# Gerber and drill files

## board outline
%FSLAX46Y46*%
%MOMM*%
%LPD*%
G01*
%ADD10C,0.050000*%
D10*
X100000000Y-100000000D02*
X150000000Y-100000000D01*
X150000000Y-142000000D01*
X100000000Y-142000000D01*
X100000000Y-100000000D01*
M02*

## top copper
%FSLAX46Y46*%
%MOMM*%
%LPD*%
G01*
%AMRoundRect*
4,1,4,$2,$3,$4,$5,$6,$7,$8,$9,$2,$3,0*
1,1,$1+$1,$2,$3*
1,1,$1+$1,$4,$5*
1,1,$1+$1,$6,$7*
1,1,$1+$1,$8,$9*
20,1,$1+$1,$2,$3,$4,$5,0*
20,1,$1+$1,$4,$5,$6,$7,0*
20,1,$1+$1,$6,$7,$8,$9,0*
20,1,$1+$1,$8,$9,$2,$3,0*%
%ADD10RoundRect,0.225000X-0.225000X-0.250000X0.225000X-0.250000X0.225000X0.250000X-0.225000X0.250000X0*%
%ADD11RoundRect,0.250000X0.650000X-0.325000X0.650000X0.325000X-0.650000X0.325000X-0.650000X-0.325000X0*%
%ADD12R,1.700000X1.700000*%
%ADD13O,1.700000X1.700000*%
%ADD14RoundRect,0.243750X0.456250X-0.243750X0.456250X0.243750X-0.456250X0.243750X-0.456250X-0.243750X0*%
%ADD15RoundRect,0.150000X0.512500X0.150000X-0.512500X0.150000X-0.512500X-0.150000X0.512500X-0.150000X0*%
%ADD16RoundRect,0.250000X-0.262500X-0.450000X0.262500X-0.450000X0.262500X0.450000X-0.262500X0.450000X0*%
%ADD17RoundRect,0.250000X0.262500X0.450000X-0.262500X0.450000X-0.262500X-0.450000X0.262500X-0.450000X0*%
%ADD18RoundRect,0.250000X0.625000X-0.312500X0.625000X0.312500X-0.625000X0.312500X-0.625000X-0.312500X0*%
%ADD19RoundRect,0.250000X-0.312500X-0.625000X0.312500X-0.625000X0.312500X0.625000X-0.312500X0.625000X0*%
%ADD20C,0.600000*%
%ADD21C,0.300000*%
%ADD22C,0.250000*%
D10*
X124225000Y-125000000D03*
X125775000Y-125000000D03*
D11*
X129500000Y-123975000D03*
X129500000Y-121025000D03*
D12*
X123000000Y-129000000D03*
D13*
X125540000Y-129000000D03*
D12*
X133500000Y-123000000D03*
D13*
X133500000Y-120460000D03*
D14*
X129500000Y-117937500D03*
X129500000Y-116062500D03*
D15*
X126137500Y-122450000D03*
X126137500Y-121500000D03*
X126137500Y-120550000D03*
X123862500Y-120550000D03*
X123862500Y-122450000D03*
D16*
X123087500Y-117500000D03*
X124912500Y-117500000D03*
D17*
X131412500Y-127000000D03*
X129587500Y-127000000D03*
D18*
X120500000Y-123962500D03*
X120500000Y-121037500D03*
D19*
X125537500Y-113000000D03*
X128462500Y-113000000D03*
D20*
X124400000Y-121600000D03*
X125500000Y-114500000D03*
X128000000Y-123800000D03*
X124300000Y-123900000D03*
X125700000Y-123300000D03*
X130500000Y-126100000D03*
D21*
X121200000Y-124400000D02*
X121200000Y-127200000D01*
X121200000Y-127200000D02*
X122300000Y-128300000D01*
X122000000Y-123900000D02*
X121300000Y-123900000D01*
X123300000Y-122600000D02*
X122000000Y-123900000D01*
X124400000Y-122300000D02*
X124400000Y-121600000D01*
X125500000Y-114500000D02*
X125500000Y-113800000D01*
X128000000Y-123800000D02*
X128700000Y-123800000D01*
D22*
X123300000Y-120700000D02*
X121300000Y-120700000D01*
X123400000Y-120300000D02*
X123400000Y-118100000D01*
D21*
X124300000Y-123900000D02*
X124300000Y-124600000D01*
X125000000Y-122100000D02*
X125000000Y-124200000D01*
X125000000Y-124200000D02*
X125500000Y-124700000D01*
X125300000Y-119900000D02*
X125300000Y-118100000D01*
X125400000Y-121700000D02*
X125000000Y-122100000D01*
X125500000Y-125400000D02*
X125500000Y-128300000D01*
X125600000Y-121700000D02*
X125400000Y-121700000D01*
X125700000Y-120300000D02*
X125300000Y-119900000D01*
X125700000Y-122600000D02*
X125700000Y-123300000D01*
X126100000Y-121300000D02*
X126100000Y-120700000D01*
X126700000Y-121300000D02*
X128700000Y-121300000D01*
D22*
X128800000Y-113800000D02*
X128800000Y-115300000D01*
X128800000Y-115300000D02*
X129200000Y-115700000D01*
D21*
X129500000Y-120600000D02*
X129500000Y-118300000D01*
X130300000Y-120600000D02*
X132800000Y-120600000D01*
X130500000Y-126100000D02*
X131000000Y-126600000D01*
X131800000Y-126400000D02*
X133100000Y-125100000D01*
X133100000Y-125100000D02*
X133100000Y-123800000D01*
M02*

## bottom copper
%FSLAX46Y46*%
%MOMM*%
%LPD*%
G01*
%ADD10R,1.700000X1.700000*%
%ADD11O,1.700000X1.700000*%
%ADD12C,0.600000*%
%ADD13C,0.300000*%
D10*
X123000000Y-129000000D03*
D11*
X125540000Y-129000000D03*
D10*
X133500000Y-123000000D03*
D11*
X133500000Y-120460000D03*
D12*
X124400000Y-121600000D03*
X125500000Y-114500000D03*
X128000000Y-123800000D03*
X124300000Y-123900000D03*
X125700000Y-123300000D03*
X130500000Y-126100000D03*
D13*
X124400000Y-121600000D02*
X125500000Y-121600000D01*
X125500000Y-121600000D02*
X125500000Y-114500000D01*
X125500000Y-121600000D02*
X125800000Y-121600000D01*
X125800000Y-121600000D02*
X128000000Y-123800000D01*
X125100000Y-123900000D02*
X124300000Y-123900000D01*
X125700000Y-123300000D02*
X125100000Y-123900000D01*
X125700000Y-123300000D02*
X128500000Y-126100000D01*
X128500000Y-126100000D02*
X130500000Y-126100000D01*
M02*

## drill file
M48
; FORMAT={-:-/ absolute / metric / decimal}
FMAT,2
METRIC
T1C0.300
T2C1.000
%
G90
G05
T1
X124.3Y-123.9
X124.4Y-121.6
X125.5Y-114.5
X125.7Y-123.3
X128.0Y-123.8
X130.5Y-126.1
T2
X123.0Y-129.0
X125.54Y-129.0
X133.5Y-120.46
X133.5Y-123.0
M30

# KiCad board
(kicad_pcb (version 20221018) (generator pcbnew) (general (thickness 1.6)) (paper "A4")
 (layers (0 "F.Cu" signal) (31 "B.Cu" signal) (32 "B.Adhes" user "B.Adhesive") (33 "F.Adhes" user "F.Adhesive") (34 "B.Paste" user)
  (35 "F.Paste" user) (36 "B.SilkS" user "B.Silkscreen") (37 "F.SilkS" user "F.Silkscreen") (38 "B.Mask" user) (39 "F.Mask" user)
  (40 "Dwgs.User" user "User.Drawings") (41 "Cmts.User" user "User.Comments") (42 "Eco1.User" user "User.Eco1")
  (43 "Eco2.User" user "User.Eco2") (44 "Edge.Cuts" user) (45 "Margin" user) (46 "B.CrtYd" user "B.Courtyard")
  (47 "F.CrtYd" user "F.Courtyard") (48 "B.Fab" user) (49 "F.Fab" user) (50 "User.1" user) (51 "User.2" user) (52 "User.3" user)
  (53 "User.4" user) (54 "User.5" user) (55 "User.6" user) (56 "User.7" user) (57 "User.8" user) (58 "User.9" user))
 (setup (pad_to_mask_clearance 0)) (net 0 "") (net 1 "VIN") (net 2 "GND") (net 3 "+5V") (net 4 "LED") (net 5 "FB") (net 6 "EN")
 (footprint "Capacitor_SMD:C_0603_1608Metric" (layer "F.Cu") (at 125 125)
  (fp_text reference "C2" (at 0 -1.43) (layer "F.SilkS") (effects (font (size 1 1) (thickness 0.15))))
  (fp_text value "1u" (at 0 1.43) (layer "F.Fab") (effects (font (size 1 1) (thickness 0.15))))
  (pad "1" smd roundrect (at -0.775 0) (size 0.9 0.95) (layers "F.Cu" "F.Paste" "F.Mask") (roundrect_rratio 0.25) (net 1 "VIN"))
  (pad "2" smd roundrect (at 0.775 0) (size 0.9 0.95) (layers "F.Cu" "F.Paste" "F.Mask") (roundrect_rratio 0.25) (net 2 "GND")))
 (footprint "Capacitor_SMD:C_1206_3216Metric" (layer "F.Cu") (at 129.5 122.5 90)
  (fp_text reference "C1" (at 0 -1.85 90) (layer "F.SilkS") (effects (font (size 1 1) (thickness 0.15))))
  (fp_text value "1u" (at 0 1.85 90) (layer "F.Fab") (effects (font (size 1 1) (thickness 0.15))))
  (pad "1" smd roundrect (at -1.475 0 90) (size 1.15 1.8) (layers "F.Cu" "F.Paste" "F.Mask") (roundrect_rratio 0.217391) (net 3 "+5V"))
  (pad "2" smd roundrect (at 1.475 0 90) (size 1.15 1.8) (layers "F.Cu" "F.Paste" "F.Mask") (roundrect_rratio 0.217391) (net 2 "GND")))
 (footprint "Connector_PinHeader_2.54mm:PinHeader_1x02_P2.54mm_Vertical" (layer "F.Cu") (at 123 129 90)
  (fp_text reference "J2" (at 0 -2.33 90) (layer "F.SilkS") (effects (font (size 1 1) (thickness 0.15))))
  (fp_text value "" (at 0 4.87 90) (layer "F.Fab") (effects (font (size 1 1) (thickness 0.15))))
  (pad "1" thru_hole rect (at 0 0 90) (size 1.7 1.7) (drill 1) (layers "*.Cu" "*.Mask") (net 3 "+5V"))
  (pad "2" thru_hole oval (at 0 2.54 90) (size 1.7 1.7) (drill 1) (layers "*.Cu" "*.Mask") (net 2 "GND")))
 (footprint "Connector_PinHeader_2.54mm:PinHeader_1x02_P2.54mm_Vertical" (layer "F.Cu") (at 133.5 123 180)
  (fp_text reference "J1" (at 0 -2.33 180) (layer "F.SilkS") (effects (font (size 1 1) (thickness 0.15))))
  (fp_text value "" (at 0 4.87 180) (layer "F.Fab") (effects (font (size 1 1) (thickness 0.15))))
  (pad "1" thru_hole rect (at 0 0 180) (size 1.7 1.7) (drill 1) (layers "*.Cu" "*.Mask") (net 1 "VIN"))
  (pad "2" thru_hole oval (at 0 2.54 180) (size 1.7 1.7) (drill 1) (layers "*.Cu" "*.Mask") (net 2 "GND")))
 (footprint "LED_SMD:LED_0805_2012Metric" (layer "F.Cu") (at 129.5 117 90)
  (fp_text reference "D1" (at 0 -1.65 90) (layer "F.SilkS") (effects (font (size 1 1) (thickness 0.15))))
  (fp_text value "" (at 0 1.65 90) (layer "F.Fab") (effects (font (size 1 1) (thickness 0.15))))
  (pad "1" smd roundrect (at -0.9375 0 90) (size 0.975 1.4) (layers "F.Cu" "F.Paste" "F.Mask") (roundrect_rratio 0.25) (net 2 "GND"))
  (pad "2" smd roundrect (at 0.9375 0 90) (size 0.975 1.4) (layers "F.Cu" "F.Paste" "F.Mask") (roundrect_rratio 0.25) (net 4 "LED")))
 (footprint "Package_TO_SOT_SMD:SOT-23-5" (layer "F.Cu") (at 125 121.5 180)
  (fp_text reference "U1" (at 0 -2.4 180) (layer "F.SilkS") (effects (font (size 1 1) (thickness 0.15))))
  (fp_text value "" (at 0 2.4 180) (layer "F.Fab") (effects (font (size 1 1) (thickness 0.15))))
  (pad "1" smd roundrect (at -1.1375 -0.95 180) (size 1.325 0.6) (layers "F.Cu" "F.Paste" "F.Mask") (roundrect_rratio 0.25) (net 1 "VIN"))
  (pad "2" smd roundrect (at -1.1375 0 180) (size 1.325 0.6) (layers "F.Cu" "F.Paste" "F.Mask") (roundrect_rratio 0.25) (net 2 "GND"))
  (pad "3" smd roundrect (at -1.1375 0.95 180) (size 1.325 0.6) (layers "F.Cu" "F.Paste" "F.Mask") (roundrect_rratio 0.25) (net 2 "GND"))
  (pad "4" smd roundrect (at 1.1375 0.95 180) (size 1.325 0.6) (layers "F.Cu" "F.Paste" "F.Mask") (roundrect_rratio 0.25) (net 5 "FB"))
  (pad "5" smd roundrect (at 1.1375 -0.95 180) (size 1.325 0.6) (layers "F.Cu" "F.Paste" "F.Mask") (roundrect_rratio 0.25) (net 3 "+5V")))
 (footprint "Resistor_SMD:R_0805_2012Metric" (layer "F.Cu") (at 124 117.5)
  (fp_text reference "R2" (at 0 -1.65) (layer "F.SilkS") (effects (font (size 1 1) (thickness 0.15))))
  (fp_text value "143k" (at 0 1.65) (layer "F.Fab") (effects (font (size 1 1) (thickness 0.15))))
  (pad "1" smd roundrect (at -0.9125 0) (size 1.025 1.4) (layers "F.Cu" "F.Paste" "F.Mask") (roundrect_rratio 0.243902) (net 5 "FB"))
  (pad "2" smd roundrect (at 0.9125 0) (size 1.025 1.4) (layers "F.Cu" "F.Paste" "F.Mask") (roundrect_rratio 0.243902) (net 2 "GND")))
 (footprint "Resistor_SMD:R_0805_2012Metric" (layer "F.Cu") (at 130.5 127 180)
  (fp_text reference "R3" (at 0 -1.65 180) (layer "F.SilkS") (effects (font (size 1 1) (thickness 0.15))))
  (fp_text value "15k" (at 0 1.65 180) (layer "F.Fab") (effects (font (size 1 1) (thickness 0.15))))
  (pad "1" smd roundrect (at -0.9125 0 180) (size 1.025 1.4) (layers "F.Cu" "F.Paste" "F.Mask") (roundrect_rratio 0.243902) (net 1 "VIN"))
  (pad "2" smd roundrect (at 0.9125 0 180) (size 1.025 1.4) (layers "F.Cu" "F.Paste" "F.Mask") (roundrect_rratio 0.243902) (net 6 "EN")))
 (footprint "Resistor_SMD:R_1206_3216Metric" (layer "F.Cu") (at 120.5 122.5 90)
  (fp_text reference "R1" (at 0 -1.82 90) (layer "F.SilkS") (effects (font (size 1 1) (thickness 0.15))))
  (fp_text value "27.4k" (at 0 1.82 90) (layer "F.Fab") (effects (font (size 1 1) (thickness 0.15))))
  (pad "1" smd roundrect (at -1.4625 0 90) (size 1.125 1.75) (layers "F.Cu" "F.Paste" "F.Mask") (roundrect_rratio 0.222222) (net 3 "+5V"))
  (pad "2" smd roundrect (at 1.4625 0 90) (size 1.125 1.75) (layers "F.Cu" "F.Paste" "F.Mask") (roundrect_rratio 0.222222) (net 5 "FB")))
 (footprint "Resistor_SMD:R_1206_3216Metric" (layer "F.Cu") (at 127 113)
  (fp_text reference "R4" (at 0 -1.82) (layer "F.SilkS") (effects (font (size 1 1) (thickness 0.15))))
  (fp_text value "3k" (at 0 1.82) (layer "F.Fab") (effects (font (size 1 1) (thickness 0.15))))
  (pad "1" smd roundrect (at -1.4625 0) (size 1.125 1.75) (layers "F.Cu" "F.Paste" "F.Mask") (roundrect_rratio 0.222222) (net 3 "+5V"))
  (pad "2" smd roundrect (at 1.4625 0) (size 1.125 1.75) (layers "F.Cu" "F.Paste" "F.Mask") (roundrect_rratio 0.222222) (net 4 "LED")))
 (gr_rect (start 100 100) (end 150 142) (stroke (width 0.05) (type default)) (fill none) (layer "Edge.Cuts"))
 (segment (start 121.2 124.4) (end 121.2 127.2) (width 0.3) (layer "F.Cu") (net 3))
 (segment (start 121.2 127.2) (end 122.3 128.3) (width 0.3) (layer "F.Cu") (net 3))
 (segment (start 122 123.9) (end 121.3 123.9) (width 0.3) (layer "F.Cu") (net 3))
 (segment (start 123.3 122.6) (end 122 123.9) (width 0.3) (layer "F.Cu") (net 3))
 (segment (start 124.4 122.3) (end 124.4 121.6) (width 0.3) (layer "F.Cu") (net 3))
 (segment (start 125.5 114.5) (end 125.5 113.8) (width 0.3) (layer "F.Cu") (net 3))
 (segment (start 128 123.8) (end 128.7 123.8) (width 0.3) (layer "F.Cu") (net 3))
 (via (at 124.4 121.6) (size 0.6) (drill 0.3) (layers "F.Cu" "B.Cu") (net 3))
 (via (at 125.5 114.5) (size 0.6) (drill 0.3) (layers "F.Cu" "B.Cu") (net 3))
 (via (at 128 123.8) (size 0.6) (drill 0.3) (layers "F.Cu" "B.Cu") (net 3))
 (segment (start 123.3 120.7) (end 121.3 120.7) (width 0.25) (layer "F.Cu") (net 5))
 (segment (start 123.4 120.3) (end 123.4 118.1) (width 0.25) (layer "F.Cu") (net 5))
 (segment (start 124.3 123.9) (end 124.3 124.6) (width 0.3) (layer "F.Cu") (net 1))
 (segment (start 124.4 121.6) (end 125.5 121.6) (width 0.3) (layer "B.Cu") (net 3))
 (segment (start 125 122.1) (end 125 124.2) (width 0.3) (layer "F.Cu") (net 2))
 (segment (start 125 124.2) (end 125.5 124.7) (width 0.3) (layer "F.Cu") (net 2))
 (segment (start 125.3 119.9) (end 125.3 118.1) (width 0.3) (layer "F.Cu") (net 2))
 (segment (start 125.4 121.7) (end 125 122.1) (width 0.3) (layer "F.Cu") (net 2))
 (segment (start 125.5 121.6) (end 125.5 114.5) (width 0.3) (layer "B.Cu") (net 3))
 (segment (start 125.5 121.6) (end 125.8 121.6) (width 0.3) (layer "B.Cu") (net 3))
 (segment (start 125.5 125.4) (end 125.5 128.3) (width 0.3) (layer "F.Cu") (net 2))
 (segment (start 125.6 121.7) (end 125.4 121.7) (width 0.3) (layer "F.Cu") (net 2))
 (segment (start 125.7 120.3) (end 125.3 119.9) (width 0.3) (layer "F.Cu") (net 2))
 (segment (start 125.7 122.6) (end 125.7 123.3) (width 0.3) (layer "F.Cu") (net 1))
 (segment (start 125.8 121.6) (end 128 123.8) (width 0.3) (layer "B.Cu") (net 3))
 (segment (start 126.1 121.3) (end 126.1 120.7) (width 0.3) (layer "F.Cu") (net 2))
 (segment (start 126.7 121.3) (end 128.7 121.3) (width 0.3) (layer "F.Cu") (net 2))
 (segment (start 128.8 113.8) (end 128.8 115.3) (width 0.25) (layer "F.Cu") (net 4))
 (segment (start 128.8 115.3) (end 129.2 115.7) (width 0.25) (layer "F.Cu") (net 4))
 (segment (start 129.5 120.6) (end 129.5 118.3) (width 0.3) (layer "F.Cu") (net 2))
 (segment (start 130.3 120.6) (end 132.8 120.6) (width 0.3) (layer "F.Cu") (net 2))
 (segment (start 130.5 126.1) (end 131 126.6) (width 0.3) (layer "F.Cu") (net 1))
 (segment (start 131.8 126.4) (end 133.1 125.1) (width 0.3) (layer "F.Cu") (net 1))
 (segment (start 133.1 125.1) (end 133.1 123.8) (width 0.3) (layer "F.Cu") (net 1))
 (via (at 124.3 123.9) (size 0.6) (drill 0.3) (layers "F.Cu" "B.Cu") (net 1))
 (via (at 125.7 123.3) (size 0.6) (drill 0.3) (layers "F.Cu" "B.Cu") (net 1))
 (via (at 130.5 126.1) (size 0.6) (drill 0.3) (layers "F.Cu" "B.Cu") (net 1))
 (segment (start 125.1 123.9) (end 124.3 123.9) (width 0.3) (layer "B.Cu") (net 1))
 (segment (start 125.7 123.3) (end 125.1 123.9) (width 0.3) (layer "B.Cu") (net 1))
 (segment (start 125.7 123.3) (end 128.5 126.1) (width 0.3) (layer "B.Cu") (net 1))
 (segment (start 128.5 126.1) (end 130.5 126.1) (width 0.3) (layer "B.Cu") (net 1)))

